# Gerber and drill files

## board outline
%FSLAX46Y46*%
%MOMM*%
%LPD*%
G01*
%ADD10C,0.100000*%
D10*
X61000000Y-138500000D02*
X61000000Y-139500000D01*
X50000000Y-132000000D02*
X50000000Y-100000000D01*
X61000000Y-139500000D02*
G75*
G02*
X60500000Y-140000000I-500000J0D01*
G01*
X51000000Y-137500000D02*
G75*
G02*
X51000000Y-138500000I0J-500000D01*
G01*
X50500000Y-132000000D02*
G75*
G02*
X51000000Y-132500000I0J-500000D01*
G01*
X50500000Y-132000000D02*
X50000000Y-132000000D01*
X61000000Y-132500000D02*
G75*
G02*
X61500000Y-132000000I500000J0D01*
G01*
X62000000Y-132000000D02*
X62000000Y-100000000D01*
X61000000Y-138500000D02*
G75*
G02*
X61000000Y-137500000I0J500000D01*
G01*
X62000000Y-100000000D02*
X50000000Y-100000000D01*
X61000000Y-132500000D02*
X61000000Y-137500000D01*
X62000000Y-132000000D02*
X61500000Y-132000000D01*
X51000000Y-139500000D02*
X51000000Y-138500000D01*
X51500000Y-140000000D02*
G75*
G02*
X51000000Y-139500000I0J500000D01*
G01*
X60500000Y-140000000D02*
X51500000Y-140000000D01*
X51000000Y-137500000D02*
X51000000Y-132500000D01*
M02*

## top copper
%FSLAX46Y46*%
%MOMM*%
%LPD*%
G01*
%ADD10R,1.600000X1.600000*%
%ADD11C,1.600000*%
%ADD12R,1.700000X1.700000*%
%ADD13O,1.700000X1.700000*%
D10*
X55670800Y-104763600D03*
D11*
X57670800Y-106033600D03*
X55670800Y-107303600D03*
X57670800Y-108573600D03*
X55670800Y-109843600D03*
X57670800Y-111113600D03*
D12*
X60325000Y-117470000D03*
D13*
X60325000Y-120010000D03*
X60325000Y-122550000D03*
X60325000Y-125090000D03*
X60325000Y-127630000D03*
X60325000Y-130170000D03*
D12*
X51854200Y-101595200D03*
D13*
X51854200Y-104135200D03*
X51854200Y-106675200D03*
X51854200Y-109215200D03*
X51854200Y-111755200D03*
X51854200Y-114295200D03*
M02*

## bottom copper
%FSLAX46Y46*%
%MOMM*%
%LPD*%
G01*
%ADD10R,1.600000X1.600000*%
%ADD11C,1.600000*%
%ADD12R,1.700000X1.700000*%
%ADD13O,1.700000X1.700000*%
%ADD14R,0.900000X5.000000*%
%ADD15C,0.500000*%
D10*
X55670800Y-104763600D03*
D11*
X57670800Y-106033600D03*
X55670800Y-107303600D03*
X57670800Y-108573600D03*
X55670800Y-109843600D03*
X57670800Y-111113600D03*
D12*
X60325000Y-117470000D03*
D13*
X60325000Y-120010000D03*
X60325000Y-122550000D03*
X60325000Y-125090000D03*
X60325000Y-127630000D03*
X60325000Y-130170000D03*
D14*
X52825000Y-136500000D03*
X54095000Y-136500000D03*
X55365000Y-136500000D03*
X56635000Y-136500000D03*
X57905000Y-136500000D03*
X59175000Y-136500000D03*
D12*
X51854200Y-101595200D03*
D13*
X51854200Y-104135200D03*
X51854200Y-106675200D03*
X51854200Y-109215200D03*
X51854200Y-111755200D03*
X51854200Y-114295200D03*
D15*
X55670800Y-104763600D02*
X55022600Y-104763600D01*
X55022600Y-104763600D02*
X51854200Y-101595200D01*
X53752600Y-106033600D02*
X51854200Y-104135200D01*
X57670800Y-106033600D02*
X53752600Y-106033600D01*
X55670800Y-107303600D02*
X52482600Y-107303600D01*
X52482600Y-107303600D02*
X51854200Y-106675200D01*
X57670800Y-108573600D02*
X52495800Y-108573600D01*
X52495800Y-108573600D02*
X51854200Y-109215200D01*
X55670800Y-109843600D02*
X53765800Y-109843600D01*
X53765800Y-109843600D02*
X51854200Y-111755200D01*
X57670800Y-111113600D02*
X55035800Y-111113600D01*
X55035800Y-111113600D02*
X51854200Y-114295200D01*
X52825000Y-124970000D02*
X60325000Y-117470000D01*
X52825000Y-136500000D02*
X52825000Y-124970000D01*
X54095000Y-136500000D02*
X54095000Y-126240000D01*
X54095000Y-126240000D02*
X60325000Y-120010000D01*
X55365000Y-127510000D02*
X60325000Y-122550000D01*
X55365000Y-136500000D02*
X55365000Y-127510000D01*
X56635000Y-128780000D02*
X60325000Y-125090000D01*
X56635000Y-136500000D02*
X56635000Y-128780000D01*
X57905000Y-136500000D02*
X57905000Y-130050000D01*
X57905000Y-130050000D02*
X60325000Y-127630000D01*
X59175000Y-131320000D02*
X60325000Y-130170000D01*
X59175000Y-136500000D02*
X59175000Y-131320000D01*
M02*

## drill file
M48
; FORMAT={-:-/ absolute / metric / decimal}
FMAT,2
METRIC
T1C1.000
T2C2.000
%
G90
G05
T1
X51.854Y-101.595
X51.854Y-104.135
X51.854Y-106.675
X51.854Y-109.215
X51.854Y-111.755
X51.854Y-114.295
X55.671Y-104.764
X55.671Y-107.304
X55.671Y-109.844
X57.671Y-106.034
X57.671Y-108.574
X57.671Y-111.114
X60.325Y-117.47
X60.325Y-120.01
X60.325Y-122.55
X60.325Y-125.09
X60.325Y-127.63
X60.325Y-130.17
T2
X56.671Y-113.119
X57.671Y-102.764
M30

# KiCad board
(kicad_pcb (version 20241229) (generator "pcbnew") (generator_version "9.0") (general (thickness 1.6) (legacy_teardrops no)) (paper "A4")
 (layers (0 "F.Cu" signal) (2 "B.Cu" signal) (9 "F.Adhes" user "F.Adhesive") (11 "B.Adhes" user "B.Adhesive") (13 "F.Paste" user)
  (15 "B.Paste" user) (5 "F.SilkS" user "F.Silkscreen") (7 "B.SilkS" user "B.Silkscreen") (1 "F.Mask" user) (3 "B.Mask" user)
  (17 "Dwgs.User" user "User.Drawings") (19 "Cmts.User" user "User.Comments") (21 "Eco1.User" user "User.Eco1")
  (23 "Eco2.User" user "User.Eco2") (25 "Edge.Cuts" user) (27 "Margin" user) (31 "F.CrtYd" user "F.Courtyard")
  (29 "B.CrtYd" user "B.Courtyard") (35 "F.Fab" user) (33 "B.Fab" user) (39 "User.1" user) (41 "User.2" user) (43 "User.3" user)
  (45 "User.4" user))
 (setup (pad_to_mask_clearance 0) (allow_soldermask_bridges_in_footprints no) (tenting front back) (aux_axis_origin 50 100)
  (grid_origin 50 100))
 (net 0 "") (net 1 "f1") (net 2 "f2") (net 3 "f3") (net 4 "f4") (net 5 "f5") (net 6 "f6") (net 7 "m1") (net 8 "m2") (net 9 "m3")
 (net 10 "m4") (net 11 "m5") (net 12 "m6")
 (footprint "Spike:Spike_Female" (layer "F.Cu") (at 55.0358 114.9236 90)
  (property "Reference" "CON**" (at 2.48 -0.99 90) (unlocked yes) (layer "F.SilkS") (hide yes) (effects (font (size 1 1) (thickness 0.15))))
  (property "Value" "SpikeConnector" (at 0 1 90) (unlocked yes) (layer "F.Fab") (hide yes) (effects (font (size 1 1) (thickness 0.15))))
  (pad "" np_thru_hole circle (at 1.805 1.635 90) (size 2.5 2.5) (drill 2) (layers))
  (pad "" np_thru_hole circle (at 12.16 2.635 90) (size 2.5 2.5) (drill 2) (layers))
  (pad "1" thru_hole rect (at 10.16 0.635 90) (size 1.6 1.6) (drill 1) (layers "*.Cu" "*.Mask") (remove_unused_layers no) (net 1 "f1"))
  (pad "2" thru_hole circle (at 8.89 2.635 90) (size 1.6 1.6) (drill 1) (layers "*.Cu" "*.Mask") (remove_unused_layers no) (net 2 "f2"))
  (pad "3" thru_hole circle (at 7.62 0.635 90) (size 1.6 1.6) (drill 1) (layers "*.Cu" "*.Mask") (remove_unused_layers no) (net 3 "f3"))
  (pad "4" thru_hole circle (at 6.35 2.635 90) (size 1.6 1.6) (drill 1) (layers "*.Cu" "*.Mask") (remove_unused_layers no) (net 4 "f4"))
  (pad "5" thru_hole circle (at 5.08 0.635 90) (size 1.6 1.6) (drill 1) (layers "*.Cu" "*.Mask") (remove_unused_layers no) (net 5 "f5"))
  (pad "6" thru_hole circle (at 3.81 2.635 90) (size 1.6 1.6) (drill 1) (layers "*.Cu" "*.Mask") (remove_unused_layers no) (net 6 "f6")))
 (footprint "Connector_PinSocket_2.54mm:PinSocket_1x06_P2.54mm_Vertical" (layer "F.Cu") (at 60.325 117.47)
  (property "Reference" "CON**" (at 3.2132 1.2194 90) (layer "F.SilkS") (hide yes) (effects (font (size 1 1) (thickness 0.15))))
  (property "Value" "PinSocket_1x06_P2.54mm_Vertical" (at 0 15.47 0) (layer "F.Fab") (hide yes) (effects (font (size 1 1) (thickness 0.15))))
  (pad "1" thru_hole rect (at 0 0) (size 1.7 1.7) (drill 1) (layers "*.Cu" "*.Mask") (remove_unused_layers no) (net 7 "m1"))
  (pad "2" thru_hole oval (at 0 2.54) (size 1.7 1.7) (drill 1) (layers "*.Cu" "*.Mask") (remove_unused_layers no) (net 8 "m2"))
  (pad "3" thru_hole oval (at 0 5.08) (size 1.7 1.7) (drill 1) (layers "*.Cu" "*.Mask") (remove_unused_layers no) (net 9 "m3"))
  (pad "4" thru_hole oval (at 0 7.62) (size 1.7 1.7) (drill 1) (layers "*.Cu" "*.Mask") (remove_unused_layers no) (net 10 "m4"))
  (pad "5" thru_hole oval (at 0 10.16) (size 1.7 1.7) (drill 1) (layers "*.Cu" "*.Mask") (remove_unused_layers no) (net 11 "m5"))
  (pad "6" thru_hole oval (at 0 12.7) (size 1.7 1.7) (drill 1) (layers "*.Cu" "*.Mask") (remove_unused_layers no) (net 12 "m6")))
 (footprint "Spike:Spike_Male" (layer "F.Cu") (at 52.825 136.5)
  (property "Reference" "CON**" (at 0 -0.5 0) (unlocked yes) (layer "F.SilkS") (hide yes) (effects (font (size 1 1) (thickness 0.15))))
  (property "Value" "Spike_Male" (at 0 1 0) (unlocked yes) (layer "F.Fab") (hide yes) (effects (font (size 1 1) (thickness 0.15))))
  (pad "1" smd rect (at 0 0) (size 0.9 5) (layers "B.Cu" "B.Mask" "B.Paste") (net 7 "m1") (thermal_bridge_angle 45))
  (pad "2" smd rect (at 1.27 0) (size 0.9 5) (layers "B.Cu" "B.Mask" "B.Paste") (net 8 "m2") (thermal_bridge_angle 45))
  (pad "3" smd rect (at 2.54 0) (size 0.9 5) (layers "B.Cu" "B.Mask" "B.Paste") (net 9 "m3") (thermal_bridge_angle 45))
  (pad "4" smd rect (at 3.81 0) (size 0.9 5) (layers "B.Cu" "B.Mask" "B.Paste") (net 10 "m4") (thermal_bridge_angle 45))
  (pad "5" smd rect (at 5.08 0) (size 0.9 5) (layers "B.Cu" "B.Mask" "B.Paste") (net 11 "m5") (thermal_bridge_angle 45))
  (pad "6" smd rect (at 6.35 0) (size 0.9 5) (layers "B.Cu" "B.Mask" "B.Paste") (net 12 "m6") (thermal_bridge_angle 45)))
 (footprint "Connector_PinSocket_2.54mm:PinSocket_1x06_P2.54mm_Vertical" (layer "F.Cu") (at 51.8542 101.5952)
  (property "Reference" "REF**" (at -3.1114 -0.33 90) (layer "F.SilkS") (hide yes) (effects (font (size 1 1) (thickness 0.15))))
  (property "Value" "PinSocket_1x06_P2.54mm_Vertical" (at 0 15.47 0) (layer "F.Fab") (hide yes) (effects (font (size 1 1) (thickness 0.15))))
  (pad "1" thru_hole rect (at 0 0) (size 1.7 1.7) (drill 1) (layers "*.Cu" "*.Mask") (remove_unused_layers no) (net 1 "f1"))
  (pad "2" thru_hole oval (at 0 2.54) (size 1.7 1.7) (drill 1) (layers "*.Cu" "*.Mask") (remove_unused_layers no) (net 2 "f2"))
  (pad "3" thru_hole oval (at 0 5.08) (size 1.7 1.7) (drill 1) (layers "*.Cu" "*.Mask") (remove_unused_layers no) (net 3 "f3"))
  (pad "4" thru_hole oval (at 0 7.62) (size 1.7 1.7) (drill 1) (layers "*.Cu" "*.Mask") (remove_unused_layers no) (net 4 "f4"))
  (pad "5" thru_hole oval (at 0 10.16) (size 1.7 1.7) (drill 1) (layers "*.Cu" "*.Mask") (remove_unused_layers no) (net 5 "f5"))
  (pad "6" thru_hole oval (at 0 12.7) (size 1.7 1.7) (drill 1) (layers "*.Cu" "*.Mask") (remove_unused_layers no) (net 6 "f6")))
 (gr_line (start 61 138.5) (end 61 139.5) (stroke (width 0.1) (type default)) (layer "Edge.Cuts"))
 (gr_line (start 50 132) (end 50 100) (stroke (width 0.1) (type default)) (layer "Edge.Cuts"))
 (gr_arc (start 61 139.5) (mid 60.853553 139.853553) (end 60.5 140) (stroke (width 0.1) (type default)) (layer "Edge.Cuts"))
 (gr_arc (start 51 137.5) (mid 51.5 138) (end 51 138.5) (stroke (width 0.1) (type default)) (layer "Edge.Cuts"))
 (gr_arc (start 50.5 132) (mid 50.853553 132.146447) (end 51 132.5) (stroke (width 0.1) (type default)) (layer "Edge.Cuts"))
 (gr_line (start 50.5 132) (end 50 132) (stroke (width 0.1) (type default)) (layer "Edge.Cuts"))
 (gr_arc (start 61 132.5) (mid 61.146447 132.146447) (end 61.5 132) (stroke (width 0.1) (type default)) (layer "Edge.Cuts"))
 (gr_line (start 62 132) (end 62 100) (stroke (width 0.1) (type solid)) (layer "Edge.Cuts"))
 (gr_arc (start 61 138.5) (mid 60.5 138) (end 61 137.5) (stroke (width 0.1) (type default)) (layer "Edge.Cuts"))
 (gr_line (start 62 100) (end 50 100) (stroke (width 0.1) (type solid)) (layer "Edge.Cuts"))
 (gr_line (start 61 132.5) (end 61 137.5) (stroke (width 0.1) (type default)) (layer "Edge.Cuts"))
 (gr_line (start 62 132) (end 61.5 132) (stroke (width 0.1) (type default)) (layer "Edge.Cuts"))
 (gr_line (start 51 139.5) (end 51 138.5) (stroke (width 0.1) (type default)) (layer "Edge.Cuts"))
 (gr_arc (start 51.5 140) (mid 51.146447 139.853553) (end 51 139.5) (stroke (width 0.1) (type default)) (layer "Edge.Cuts"))
 (gr_line (start 60.5 140) (end 51.5 140) (stroke (width 0.1) (type default)) (layer "Edge.Cuts"))
 (gr_line (start 51 137.5) (end 51 132.5) (stroke (width 0.1) (type default)) (layer "Edge.Cuts"))
 (segment (start 55.6708 104.7636) (end 55.0226 104.7636) (width 0.5) (layer "B.Cu") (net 1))
 (segment (start 55.0226 104.7636) (end 51.8542 101.5952) (width 0.5) (layer "B.Cu") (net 1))
 (segment (start 53.7526 106.0336) (end 51.8542 104.1352) (width 0.5) (layer "B.Cu") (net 2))
 (segment (start 57.6708 106.0336) (end 53.7526 106.0336) (width 0.5) (layer "B.Cu") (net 2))
 (segment (start 55.6708 107.3036) (end 52.4826 107.3036) (width 0.5) (layer "B.Cu") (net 3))
 (segment (start 52.4826 107.3036) (end 51.8542 106.6752) (width 0.5) (layer "B.Cu") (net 3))
 (segment (start 57.6708 108.5736) (end 52.4958 108.5736) (width 0.5) (layer "B.Cu") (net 4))
 (segment (start 52.4958 108.5736) (end 51.8542 109.2152) (width 0.5) (layer "B.Cu") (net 4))
 (segment (start 55.6708 109.8436) (end 53.7658 109.8436) (width 0.5) (layer "B.Cu") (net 5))
 (segment (start 53.7658 109.8436) (end 51.8542 111.7552) (width 0.5) (layer "B.Cu") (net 5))
 (segment (start 57.6708 111.1136) (end 55.0358 111.1136) (width 0.5) (layer "B.Cu") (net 6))
 (segment (start 55.0358 111.1136) (end 51.8542 114.2952) (width 0.5) (layer "B.Cu") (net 6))
 (segment (start 52.825 124.97) (end 60.325 117.47) (width 0.5) (layer "B.Cu") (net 7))
 (segment (start 52.825 136.5) (end 52.825 124.97) (width 0.5) (layer "B.Cu") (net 7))
 (segment (start 54.095 136.5) (end 54.095 126.24) (width 0.5) (layer "B.Cu") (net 8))
 (segment (start 54.095 126.24) (end 60.325 120.01) (width 0.5) (layer "B.Cu") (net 8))
 (segment (start 55.365 127.51) (end 60.325 122.55) (width 0.5) (layer "B.Cu") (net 9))
 (segment (start 55.365 136.5) (end 55.365 127.51) (width 0.5) (layer "B.Cu") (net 9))
 (segment (start 56.635 128.78) (end 60.325 125.09) (width 0.5) (layer "B.Cu") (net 10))
 (segment (start 56.635 136.5) (end 56.635 128.78) (width 0.5) (layer "B.Cu") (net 10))
 (segment (start 57.905 136.5) (end 57.905 130.05) (width 0.5) (layer "B.Cu") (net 11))
 (segment (start 57.905 130.05) (end 60.325 127.63) (width 0.5) (layer "B.Cu") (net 11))
 (segment (start 59.175 131.32) (end 60.325 130.17) (width 0.5) (layer "B.Cu") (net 12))
 (segment (start 59.175 136.5) (end 59.175 131.32) (width 0.5) (layer "B.Cu") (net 12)))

